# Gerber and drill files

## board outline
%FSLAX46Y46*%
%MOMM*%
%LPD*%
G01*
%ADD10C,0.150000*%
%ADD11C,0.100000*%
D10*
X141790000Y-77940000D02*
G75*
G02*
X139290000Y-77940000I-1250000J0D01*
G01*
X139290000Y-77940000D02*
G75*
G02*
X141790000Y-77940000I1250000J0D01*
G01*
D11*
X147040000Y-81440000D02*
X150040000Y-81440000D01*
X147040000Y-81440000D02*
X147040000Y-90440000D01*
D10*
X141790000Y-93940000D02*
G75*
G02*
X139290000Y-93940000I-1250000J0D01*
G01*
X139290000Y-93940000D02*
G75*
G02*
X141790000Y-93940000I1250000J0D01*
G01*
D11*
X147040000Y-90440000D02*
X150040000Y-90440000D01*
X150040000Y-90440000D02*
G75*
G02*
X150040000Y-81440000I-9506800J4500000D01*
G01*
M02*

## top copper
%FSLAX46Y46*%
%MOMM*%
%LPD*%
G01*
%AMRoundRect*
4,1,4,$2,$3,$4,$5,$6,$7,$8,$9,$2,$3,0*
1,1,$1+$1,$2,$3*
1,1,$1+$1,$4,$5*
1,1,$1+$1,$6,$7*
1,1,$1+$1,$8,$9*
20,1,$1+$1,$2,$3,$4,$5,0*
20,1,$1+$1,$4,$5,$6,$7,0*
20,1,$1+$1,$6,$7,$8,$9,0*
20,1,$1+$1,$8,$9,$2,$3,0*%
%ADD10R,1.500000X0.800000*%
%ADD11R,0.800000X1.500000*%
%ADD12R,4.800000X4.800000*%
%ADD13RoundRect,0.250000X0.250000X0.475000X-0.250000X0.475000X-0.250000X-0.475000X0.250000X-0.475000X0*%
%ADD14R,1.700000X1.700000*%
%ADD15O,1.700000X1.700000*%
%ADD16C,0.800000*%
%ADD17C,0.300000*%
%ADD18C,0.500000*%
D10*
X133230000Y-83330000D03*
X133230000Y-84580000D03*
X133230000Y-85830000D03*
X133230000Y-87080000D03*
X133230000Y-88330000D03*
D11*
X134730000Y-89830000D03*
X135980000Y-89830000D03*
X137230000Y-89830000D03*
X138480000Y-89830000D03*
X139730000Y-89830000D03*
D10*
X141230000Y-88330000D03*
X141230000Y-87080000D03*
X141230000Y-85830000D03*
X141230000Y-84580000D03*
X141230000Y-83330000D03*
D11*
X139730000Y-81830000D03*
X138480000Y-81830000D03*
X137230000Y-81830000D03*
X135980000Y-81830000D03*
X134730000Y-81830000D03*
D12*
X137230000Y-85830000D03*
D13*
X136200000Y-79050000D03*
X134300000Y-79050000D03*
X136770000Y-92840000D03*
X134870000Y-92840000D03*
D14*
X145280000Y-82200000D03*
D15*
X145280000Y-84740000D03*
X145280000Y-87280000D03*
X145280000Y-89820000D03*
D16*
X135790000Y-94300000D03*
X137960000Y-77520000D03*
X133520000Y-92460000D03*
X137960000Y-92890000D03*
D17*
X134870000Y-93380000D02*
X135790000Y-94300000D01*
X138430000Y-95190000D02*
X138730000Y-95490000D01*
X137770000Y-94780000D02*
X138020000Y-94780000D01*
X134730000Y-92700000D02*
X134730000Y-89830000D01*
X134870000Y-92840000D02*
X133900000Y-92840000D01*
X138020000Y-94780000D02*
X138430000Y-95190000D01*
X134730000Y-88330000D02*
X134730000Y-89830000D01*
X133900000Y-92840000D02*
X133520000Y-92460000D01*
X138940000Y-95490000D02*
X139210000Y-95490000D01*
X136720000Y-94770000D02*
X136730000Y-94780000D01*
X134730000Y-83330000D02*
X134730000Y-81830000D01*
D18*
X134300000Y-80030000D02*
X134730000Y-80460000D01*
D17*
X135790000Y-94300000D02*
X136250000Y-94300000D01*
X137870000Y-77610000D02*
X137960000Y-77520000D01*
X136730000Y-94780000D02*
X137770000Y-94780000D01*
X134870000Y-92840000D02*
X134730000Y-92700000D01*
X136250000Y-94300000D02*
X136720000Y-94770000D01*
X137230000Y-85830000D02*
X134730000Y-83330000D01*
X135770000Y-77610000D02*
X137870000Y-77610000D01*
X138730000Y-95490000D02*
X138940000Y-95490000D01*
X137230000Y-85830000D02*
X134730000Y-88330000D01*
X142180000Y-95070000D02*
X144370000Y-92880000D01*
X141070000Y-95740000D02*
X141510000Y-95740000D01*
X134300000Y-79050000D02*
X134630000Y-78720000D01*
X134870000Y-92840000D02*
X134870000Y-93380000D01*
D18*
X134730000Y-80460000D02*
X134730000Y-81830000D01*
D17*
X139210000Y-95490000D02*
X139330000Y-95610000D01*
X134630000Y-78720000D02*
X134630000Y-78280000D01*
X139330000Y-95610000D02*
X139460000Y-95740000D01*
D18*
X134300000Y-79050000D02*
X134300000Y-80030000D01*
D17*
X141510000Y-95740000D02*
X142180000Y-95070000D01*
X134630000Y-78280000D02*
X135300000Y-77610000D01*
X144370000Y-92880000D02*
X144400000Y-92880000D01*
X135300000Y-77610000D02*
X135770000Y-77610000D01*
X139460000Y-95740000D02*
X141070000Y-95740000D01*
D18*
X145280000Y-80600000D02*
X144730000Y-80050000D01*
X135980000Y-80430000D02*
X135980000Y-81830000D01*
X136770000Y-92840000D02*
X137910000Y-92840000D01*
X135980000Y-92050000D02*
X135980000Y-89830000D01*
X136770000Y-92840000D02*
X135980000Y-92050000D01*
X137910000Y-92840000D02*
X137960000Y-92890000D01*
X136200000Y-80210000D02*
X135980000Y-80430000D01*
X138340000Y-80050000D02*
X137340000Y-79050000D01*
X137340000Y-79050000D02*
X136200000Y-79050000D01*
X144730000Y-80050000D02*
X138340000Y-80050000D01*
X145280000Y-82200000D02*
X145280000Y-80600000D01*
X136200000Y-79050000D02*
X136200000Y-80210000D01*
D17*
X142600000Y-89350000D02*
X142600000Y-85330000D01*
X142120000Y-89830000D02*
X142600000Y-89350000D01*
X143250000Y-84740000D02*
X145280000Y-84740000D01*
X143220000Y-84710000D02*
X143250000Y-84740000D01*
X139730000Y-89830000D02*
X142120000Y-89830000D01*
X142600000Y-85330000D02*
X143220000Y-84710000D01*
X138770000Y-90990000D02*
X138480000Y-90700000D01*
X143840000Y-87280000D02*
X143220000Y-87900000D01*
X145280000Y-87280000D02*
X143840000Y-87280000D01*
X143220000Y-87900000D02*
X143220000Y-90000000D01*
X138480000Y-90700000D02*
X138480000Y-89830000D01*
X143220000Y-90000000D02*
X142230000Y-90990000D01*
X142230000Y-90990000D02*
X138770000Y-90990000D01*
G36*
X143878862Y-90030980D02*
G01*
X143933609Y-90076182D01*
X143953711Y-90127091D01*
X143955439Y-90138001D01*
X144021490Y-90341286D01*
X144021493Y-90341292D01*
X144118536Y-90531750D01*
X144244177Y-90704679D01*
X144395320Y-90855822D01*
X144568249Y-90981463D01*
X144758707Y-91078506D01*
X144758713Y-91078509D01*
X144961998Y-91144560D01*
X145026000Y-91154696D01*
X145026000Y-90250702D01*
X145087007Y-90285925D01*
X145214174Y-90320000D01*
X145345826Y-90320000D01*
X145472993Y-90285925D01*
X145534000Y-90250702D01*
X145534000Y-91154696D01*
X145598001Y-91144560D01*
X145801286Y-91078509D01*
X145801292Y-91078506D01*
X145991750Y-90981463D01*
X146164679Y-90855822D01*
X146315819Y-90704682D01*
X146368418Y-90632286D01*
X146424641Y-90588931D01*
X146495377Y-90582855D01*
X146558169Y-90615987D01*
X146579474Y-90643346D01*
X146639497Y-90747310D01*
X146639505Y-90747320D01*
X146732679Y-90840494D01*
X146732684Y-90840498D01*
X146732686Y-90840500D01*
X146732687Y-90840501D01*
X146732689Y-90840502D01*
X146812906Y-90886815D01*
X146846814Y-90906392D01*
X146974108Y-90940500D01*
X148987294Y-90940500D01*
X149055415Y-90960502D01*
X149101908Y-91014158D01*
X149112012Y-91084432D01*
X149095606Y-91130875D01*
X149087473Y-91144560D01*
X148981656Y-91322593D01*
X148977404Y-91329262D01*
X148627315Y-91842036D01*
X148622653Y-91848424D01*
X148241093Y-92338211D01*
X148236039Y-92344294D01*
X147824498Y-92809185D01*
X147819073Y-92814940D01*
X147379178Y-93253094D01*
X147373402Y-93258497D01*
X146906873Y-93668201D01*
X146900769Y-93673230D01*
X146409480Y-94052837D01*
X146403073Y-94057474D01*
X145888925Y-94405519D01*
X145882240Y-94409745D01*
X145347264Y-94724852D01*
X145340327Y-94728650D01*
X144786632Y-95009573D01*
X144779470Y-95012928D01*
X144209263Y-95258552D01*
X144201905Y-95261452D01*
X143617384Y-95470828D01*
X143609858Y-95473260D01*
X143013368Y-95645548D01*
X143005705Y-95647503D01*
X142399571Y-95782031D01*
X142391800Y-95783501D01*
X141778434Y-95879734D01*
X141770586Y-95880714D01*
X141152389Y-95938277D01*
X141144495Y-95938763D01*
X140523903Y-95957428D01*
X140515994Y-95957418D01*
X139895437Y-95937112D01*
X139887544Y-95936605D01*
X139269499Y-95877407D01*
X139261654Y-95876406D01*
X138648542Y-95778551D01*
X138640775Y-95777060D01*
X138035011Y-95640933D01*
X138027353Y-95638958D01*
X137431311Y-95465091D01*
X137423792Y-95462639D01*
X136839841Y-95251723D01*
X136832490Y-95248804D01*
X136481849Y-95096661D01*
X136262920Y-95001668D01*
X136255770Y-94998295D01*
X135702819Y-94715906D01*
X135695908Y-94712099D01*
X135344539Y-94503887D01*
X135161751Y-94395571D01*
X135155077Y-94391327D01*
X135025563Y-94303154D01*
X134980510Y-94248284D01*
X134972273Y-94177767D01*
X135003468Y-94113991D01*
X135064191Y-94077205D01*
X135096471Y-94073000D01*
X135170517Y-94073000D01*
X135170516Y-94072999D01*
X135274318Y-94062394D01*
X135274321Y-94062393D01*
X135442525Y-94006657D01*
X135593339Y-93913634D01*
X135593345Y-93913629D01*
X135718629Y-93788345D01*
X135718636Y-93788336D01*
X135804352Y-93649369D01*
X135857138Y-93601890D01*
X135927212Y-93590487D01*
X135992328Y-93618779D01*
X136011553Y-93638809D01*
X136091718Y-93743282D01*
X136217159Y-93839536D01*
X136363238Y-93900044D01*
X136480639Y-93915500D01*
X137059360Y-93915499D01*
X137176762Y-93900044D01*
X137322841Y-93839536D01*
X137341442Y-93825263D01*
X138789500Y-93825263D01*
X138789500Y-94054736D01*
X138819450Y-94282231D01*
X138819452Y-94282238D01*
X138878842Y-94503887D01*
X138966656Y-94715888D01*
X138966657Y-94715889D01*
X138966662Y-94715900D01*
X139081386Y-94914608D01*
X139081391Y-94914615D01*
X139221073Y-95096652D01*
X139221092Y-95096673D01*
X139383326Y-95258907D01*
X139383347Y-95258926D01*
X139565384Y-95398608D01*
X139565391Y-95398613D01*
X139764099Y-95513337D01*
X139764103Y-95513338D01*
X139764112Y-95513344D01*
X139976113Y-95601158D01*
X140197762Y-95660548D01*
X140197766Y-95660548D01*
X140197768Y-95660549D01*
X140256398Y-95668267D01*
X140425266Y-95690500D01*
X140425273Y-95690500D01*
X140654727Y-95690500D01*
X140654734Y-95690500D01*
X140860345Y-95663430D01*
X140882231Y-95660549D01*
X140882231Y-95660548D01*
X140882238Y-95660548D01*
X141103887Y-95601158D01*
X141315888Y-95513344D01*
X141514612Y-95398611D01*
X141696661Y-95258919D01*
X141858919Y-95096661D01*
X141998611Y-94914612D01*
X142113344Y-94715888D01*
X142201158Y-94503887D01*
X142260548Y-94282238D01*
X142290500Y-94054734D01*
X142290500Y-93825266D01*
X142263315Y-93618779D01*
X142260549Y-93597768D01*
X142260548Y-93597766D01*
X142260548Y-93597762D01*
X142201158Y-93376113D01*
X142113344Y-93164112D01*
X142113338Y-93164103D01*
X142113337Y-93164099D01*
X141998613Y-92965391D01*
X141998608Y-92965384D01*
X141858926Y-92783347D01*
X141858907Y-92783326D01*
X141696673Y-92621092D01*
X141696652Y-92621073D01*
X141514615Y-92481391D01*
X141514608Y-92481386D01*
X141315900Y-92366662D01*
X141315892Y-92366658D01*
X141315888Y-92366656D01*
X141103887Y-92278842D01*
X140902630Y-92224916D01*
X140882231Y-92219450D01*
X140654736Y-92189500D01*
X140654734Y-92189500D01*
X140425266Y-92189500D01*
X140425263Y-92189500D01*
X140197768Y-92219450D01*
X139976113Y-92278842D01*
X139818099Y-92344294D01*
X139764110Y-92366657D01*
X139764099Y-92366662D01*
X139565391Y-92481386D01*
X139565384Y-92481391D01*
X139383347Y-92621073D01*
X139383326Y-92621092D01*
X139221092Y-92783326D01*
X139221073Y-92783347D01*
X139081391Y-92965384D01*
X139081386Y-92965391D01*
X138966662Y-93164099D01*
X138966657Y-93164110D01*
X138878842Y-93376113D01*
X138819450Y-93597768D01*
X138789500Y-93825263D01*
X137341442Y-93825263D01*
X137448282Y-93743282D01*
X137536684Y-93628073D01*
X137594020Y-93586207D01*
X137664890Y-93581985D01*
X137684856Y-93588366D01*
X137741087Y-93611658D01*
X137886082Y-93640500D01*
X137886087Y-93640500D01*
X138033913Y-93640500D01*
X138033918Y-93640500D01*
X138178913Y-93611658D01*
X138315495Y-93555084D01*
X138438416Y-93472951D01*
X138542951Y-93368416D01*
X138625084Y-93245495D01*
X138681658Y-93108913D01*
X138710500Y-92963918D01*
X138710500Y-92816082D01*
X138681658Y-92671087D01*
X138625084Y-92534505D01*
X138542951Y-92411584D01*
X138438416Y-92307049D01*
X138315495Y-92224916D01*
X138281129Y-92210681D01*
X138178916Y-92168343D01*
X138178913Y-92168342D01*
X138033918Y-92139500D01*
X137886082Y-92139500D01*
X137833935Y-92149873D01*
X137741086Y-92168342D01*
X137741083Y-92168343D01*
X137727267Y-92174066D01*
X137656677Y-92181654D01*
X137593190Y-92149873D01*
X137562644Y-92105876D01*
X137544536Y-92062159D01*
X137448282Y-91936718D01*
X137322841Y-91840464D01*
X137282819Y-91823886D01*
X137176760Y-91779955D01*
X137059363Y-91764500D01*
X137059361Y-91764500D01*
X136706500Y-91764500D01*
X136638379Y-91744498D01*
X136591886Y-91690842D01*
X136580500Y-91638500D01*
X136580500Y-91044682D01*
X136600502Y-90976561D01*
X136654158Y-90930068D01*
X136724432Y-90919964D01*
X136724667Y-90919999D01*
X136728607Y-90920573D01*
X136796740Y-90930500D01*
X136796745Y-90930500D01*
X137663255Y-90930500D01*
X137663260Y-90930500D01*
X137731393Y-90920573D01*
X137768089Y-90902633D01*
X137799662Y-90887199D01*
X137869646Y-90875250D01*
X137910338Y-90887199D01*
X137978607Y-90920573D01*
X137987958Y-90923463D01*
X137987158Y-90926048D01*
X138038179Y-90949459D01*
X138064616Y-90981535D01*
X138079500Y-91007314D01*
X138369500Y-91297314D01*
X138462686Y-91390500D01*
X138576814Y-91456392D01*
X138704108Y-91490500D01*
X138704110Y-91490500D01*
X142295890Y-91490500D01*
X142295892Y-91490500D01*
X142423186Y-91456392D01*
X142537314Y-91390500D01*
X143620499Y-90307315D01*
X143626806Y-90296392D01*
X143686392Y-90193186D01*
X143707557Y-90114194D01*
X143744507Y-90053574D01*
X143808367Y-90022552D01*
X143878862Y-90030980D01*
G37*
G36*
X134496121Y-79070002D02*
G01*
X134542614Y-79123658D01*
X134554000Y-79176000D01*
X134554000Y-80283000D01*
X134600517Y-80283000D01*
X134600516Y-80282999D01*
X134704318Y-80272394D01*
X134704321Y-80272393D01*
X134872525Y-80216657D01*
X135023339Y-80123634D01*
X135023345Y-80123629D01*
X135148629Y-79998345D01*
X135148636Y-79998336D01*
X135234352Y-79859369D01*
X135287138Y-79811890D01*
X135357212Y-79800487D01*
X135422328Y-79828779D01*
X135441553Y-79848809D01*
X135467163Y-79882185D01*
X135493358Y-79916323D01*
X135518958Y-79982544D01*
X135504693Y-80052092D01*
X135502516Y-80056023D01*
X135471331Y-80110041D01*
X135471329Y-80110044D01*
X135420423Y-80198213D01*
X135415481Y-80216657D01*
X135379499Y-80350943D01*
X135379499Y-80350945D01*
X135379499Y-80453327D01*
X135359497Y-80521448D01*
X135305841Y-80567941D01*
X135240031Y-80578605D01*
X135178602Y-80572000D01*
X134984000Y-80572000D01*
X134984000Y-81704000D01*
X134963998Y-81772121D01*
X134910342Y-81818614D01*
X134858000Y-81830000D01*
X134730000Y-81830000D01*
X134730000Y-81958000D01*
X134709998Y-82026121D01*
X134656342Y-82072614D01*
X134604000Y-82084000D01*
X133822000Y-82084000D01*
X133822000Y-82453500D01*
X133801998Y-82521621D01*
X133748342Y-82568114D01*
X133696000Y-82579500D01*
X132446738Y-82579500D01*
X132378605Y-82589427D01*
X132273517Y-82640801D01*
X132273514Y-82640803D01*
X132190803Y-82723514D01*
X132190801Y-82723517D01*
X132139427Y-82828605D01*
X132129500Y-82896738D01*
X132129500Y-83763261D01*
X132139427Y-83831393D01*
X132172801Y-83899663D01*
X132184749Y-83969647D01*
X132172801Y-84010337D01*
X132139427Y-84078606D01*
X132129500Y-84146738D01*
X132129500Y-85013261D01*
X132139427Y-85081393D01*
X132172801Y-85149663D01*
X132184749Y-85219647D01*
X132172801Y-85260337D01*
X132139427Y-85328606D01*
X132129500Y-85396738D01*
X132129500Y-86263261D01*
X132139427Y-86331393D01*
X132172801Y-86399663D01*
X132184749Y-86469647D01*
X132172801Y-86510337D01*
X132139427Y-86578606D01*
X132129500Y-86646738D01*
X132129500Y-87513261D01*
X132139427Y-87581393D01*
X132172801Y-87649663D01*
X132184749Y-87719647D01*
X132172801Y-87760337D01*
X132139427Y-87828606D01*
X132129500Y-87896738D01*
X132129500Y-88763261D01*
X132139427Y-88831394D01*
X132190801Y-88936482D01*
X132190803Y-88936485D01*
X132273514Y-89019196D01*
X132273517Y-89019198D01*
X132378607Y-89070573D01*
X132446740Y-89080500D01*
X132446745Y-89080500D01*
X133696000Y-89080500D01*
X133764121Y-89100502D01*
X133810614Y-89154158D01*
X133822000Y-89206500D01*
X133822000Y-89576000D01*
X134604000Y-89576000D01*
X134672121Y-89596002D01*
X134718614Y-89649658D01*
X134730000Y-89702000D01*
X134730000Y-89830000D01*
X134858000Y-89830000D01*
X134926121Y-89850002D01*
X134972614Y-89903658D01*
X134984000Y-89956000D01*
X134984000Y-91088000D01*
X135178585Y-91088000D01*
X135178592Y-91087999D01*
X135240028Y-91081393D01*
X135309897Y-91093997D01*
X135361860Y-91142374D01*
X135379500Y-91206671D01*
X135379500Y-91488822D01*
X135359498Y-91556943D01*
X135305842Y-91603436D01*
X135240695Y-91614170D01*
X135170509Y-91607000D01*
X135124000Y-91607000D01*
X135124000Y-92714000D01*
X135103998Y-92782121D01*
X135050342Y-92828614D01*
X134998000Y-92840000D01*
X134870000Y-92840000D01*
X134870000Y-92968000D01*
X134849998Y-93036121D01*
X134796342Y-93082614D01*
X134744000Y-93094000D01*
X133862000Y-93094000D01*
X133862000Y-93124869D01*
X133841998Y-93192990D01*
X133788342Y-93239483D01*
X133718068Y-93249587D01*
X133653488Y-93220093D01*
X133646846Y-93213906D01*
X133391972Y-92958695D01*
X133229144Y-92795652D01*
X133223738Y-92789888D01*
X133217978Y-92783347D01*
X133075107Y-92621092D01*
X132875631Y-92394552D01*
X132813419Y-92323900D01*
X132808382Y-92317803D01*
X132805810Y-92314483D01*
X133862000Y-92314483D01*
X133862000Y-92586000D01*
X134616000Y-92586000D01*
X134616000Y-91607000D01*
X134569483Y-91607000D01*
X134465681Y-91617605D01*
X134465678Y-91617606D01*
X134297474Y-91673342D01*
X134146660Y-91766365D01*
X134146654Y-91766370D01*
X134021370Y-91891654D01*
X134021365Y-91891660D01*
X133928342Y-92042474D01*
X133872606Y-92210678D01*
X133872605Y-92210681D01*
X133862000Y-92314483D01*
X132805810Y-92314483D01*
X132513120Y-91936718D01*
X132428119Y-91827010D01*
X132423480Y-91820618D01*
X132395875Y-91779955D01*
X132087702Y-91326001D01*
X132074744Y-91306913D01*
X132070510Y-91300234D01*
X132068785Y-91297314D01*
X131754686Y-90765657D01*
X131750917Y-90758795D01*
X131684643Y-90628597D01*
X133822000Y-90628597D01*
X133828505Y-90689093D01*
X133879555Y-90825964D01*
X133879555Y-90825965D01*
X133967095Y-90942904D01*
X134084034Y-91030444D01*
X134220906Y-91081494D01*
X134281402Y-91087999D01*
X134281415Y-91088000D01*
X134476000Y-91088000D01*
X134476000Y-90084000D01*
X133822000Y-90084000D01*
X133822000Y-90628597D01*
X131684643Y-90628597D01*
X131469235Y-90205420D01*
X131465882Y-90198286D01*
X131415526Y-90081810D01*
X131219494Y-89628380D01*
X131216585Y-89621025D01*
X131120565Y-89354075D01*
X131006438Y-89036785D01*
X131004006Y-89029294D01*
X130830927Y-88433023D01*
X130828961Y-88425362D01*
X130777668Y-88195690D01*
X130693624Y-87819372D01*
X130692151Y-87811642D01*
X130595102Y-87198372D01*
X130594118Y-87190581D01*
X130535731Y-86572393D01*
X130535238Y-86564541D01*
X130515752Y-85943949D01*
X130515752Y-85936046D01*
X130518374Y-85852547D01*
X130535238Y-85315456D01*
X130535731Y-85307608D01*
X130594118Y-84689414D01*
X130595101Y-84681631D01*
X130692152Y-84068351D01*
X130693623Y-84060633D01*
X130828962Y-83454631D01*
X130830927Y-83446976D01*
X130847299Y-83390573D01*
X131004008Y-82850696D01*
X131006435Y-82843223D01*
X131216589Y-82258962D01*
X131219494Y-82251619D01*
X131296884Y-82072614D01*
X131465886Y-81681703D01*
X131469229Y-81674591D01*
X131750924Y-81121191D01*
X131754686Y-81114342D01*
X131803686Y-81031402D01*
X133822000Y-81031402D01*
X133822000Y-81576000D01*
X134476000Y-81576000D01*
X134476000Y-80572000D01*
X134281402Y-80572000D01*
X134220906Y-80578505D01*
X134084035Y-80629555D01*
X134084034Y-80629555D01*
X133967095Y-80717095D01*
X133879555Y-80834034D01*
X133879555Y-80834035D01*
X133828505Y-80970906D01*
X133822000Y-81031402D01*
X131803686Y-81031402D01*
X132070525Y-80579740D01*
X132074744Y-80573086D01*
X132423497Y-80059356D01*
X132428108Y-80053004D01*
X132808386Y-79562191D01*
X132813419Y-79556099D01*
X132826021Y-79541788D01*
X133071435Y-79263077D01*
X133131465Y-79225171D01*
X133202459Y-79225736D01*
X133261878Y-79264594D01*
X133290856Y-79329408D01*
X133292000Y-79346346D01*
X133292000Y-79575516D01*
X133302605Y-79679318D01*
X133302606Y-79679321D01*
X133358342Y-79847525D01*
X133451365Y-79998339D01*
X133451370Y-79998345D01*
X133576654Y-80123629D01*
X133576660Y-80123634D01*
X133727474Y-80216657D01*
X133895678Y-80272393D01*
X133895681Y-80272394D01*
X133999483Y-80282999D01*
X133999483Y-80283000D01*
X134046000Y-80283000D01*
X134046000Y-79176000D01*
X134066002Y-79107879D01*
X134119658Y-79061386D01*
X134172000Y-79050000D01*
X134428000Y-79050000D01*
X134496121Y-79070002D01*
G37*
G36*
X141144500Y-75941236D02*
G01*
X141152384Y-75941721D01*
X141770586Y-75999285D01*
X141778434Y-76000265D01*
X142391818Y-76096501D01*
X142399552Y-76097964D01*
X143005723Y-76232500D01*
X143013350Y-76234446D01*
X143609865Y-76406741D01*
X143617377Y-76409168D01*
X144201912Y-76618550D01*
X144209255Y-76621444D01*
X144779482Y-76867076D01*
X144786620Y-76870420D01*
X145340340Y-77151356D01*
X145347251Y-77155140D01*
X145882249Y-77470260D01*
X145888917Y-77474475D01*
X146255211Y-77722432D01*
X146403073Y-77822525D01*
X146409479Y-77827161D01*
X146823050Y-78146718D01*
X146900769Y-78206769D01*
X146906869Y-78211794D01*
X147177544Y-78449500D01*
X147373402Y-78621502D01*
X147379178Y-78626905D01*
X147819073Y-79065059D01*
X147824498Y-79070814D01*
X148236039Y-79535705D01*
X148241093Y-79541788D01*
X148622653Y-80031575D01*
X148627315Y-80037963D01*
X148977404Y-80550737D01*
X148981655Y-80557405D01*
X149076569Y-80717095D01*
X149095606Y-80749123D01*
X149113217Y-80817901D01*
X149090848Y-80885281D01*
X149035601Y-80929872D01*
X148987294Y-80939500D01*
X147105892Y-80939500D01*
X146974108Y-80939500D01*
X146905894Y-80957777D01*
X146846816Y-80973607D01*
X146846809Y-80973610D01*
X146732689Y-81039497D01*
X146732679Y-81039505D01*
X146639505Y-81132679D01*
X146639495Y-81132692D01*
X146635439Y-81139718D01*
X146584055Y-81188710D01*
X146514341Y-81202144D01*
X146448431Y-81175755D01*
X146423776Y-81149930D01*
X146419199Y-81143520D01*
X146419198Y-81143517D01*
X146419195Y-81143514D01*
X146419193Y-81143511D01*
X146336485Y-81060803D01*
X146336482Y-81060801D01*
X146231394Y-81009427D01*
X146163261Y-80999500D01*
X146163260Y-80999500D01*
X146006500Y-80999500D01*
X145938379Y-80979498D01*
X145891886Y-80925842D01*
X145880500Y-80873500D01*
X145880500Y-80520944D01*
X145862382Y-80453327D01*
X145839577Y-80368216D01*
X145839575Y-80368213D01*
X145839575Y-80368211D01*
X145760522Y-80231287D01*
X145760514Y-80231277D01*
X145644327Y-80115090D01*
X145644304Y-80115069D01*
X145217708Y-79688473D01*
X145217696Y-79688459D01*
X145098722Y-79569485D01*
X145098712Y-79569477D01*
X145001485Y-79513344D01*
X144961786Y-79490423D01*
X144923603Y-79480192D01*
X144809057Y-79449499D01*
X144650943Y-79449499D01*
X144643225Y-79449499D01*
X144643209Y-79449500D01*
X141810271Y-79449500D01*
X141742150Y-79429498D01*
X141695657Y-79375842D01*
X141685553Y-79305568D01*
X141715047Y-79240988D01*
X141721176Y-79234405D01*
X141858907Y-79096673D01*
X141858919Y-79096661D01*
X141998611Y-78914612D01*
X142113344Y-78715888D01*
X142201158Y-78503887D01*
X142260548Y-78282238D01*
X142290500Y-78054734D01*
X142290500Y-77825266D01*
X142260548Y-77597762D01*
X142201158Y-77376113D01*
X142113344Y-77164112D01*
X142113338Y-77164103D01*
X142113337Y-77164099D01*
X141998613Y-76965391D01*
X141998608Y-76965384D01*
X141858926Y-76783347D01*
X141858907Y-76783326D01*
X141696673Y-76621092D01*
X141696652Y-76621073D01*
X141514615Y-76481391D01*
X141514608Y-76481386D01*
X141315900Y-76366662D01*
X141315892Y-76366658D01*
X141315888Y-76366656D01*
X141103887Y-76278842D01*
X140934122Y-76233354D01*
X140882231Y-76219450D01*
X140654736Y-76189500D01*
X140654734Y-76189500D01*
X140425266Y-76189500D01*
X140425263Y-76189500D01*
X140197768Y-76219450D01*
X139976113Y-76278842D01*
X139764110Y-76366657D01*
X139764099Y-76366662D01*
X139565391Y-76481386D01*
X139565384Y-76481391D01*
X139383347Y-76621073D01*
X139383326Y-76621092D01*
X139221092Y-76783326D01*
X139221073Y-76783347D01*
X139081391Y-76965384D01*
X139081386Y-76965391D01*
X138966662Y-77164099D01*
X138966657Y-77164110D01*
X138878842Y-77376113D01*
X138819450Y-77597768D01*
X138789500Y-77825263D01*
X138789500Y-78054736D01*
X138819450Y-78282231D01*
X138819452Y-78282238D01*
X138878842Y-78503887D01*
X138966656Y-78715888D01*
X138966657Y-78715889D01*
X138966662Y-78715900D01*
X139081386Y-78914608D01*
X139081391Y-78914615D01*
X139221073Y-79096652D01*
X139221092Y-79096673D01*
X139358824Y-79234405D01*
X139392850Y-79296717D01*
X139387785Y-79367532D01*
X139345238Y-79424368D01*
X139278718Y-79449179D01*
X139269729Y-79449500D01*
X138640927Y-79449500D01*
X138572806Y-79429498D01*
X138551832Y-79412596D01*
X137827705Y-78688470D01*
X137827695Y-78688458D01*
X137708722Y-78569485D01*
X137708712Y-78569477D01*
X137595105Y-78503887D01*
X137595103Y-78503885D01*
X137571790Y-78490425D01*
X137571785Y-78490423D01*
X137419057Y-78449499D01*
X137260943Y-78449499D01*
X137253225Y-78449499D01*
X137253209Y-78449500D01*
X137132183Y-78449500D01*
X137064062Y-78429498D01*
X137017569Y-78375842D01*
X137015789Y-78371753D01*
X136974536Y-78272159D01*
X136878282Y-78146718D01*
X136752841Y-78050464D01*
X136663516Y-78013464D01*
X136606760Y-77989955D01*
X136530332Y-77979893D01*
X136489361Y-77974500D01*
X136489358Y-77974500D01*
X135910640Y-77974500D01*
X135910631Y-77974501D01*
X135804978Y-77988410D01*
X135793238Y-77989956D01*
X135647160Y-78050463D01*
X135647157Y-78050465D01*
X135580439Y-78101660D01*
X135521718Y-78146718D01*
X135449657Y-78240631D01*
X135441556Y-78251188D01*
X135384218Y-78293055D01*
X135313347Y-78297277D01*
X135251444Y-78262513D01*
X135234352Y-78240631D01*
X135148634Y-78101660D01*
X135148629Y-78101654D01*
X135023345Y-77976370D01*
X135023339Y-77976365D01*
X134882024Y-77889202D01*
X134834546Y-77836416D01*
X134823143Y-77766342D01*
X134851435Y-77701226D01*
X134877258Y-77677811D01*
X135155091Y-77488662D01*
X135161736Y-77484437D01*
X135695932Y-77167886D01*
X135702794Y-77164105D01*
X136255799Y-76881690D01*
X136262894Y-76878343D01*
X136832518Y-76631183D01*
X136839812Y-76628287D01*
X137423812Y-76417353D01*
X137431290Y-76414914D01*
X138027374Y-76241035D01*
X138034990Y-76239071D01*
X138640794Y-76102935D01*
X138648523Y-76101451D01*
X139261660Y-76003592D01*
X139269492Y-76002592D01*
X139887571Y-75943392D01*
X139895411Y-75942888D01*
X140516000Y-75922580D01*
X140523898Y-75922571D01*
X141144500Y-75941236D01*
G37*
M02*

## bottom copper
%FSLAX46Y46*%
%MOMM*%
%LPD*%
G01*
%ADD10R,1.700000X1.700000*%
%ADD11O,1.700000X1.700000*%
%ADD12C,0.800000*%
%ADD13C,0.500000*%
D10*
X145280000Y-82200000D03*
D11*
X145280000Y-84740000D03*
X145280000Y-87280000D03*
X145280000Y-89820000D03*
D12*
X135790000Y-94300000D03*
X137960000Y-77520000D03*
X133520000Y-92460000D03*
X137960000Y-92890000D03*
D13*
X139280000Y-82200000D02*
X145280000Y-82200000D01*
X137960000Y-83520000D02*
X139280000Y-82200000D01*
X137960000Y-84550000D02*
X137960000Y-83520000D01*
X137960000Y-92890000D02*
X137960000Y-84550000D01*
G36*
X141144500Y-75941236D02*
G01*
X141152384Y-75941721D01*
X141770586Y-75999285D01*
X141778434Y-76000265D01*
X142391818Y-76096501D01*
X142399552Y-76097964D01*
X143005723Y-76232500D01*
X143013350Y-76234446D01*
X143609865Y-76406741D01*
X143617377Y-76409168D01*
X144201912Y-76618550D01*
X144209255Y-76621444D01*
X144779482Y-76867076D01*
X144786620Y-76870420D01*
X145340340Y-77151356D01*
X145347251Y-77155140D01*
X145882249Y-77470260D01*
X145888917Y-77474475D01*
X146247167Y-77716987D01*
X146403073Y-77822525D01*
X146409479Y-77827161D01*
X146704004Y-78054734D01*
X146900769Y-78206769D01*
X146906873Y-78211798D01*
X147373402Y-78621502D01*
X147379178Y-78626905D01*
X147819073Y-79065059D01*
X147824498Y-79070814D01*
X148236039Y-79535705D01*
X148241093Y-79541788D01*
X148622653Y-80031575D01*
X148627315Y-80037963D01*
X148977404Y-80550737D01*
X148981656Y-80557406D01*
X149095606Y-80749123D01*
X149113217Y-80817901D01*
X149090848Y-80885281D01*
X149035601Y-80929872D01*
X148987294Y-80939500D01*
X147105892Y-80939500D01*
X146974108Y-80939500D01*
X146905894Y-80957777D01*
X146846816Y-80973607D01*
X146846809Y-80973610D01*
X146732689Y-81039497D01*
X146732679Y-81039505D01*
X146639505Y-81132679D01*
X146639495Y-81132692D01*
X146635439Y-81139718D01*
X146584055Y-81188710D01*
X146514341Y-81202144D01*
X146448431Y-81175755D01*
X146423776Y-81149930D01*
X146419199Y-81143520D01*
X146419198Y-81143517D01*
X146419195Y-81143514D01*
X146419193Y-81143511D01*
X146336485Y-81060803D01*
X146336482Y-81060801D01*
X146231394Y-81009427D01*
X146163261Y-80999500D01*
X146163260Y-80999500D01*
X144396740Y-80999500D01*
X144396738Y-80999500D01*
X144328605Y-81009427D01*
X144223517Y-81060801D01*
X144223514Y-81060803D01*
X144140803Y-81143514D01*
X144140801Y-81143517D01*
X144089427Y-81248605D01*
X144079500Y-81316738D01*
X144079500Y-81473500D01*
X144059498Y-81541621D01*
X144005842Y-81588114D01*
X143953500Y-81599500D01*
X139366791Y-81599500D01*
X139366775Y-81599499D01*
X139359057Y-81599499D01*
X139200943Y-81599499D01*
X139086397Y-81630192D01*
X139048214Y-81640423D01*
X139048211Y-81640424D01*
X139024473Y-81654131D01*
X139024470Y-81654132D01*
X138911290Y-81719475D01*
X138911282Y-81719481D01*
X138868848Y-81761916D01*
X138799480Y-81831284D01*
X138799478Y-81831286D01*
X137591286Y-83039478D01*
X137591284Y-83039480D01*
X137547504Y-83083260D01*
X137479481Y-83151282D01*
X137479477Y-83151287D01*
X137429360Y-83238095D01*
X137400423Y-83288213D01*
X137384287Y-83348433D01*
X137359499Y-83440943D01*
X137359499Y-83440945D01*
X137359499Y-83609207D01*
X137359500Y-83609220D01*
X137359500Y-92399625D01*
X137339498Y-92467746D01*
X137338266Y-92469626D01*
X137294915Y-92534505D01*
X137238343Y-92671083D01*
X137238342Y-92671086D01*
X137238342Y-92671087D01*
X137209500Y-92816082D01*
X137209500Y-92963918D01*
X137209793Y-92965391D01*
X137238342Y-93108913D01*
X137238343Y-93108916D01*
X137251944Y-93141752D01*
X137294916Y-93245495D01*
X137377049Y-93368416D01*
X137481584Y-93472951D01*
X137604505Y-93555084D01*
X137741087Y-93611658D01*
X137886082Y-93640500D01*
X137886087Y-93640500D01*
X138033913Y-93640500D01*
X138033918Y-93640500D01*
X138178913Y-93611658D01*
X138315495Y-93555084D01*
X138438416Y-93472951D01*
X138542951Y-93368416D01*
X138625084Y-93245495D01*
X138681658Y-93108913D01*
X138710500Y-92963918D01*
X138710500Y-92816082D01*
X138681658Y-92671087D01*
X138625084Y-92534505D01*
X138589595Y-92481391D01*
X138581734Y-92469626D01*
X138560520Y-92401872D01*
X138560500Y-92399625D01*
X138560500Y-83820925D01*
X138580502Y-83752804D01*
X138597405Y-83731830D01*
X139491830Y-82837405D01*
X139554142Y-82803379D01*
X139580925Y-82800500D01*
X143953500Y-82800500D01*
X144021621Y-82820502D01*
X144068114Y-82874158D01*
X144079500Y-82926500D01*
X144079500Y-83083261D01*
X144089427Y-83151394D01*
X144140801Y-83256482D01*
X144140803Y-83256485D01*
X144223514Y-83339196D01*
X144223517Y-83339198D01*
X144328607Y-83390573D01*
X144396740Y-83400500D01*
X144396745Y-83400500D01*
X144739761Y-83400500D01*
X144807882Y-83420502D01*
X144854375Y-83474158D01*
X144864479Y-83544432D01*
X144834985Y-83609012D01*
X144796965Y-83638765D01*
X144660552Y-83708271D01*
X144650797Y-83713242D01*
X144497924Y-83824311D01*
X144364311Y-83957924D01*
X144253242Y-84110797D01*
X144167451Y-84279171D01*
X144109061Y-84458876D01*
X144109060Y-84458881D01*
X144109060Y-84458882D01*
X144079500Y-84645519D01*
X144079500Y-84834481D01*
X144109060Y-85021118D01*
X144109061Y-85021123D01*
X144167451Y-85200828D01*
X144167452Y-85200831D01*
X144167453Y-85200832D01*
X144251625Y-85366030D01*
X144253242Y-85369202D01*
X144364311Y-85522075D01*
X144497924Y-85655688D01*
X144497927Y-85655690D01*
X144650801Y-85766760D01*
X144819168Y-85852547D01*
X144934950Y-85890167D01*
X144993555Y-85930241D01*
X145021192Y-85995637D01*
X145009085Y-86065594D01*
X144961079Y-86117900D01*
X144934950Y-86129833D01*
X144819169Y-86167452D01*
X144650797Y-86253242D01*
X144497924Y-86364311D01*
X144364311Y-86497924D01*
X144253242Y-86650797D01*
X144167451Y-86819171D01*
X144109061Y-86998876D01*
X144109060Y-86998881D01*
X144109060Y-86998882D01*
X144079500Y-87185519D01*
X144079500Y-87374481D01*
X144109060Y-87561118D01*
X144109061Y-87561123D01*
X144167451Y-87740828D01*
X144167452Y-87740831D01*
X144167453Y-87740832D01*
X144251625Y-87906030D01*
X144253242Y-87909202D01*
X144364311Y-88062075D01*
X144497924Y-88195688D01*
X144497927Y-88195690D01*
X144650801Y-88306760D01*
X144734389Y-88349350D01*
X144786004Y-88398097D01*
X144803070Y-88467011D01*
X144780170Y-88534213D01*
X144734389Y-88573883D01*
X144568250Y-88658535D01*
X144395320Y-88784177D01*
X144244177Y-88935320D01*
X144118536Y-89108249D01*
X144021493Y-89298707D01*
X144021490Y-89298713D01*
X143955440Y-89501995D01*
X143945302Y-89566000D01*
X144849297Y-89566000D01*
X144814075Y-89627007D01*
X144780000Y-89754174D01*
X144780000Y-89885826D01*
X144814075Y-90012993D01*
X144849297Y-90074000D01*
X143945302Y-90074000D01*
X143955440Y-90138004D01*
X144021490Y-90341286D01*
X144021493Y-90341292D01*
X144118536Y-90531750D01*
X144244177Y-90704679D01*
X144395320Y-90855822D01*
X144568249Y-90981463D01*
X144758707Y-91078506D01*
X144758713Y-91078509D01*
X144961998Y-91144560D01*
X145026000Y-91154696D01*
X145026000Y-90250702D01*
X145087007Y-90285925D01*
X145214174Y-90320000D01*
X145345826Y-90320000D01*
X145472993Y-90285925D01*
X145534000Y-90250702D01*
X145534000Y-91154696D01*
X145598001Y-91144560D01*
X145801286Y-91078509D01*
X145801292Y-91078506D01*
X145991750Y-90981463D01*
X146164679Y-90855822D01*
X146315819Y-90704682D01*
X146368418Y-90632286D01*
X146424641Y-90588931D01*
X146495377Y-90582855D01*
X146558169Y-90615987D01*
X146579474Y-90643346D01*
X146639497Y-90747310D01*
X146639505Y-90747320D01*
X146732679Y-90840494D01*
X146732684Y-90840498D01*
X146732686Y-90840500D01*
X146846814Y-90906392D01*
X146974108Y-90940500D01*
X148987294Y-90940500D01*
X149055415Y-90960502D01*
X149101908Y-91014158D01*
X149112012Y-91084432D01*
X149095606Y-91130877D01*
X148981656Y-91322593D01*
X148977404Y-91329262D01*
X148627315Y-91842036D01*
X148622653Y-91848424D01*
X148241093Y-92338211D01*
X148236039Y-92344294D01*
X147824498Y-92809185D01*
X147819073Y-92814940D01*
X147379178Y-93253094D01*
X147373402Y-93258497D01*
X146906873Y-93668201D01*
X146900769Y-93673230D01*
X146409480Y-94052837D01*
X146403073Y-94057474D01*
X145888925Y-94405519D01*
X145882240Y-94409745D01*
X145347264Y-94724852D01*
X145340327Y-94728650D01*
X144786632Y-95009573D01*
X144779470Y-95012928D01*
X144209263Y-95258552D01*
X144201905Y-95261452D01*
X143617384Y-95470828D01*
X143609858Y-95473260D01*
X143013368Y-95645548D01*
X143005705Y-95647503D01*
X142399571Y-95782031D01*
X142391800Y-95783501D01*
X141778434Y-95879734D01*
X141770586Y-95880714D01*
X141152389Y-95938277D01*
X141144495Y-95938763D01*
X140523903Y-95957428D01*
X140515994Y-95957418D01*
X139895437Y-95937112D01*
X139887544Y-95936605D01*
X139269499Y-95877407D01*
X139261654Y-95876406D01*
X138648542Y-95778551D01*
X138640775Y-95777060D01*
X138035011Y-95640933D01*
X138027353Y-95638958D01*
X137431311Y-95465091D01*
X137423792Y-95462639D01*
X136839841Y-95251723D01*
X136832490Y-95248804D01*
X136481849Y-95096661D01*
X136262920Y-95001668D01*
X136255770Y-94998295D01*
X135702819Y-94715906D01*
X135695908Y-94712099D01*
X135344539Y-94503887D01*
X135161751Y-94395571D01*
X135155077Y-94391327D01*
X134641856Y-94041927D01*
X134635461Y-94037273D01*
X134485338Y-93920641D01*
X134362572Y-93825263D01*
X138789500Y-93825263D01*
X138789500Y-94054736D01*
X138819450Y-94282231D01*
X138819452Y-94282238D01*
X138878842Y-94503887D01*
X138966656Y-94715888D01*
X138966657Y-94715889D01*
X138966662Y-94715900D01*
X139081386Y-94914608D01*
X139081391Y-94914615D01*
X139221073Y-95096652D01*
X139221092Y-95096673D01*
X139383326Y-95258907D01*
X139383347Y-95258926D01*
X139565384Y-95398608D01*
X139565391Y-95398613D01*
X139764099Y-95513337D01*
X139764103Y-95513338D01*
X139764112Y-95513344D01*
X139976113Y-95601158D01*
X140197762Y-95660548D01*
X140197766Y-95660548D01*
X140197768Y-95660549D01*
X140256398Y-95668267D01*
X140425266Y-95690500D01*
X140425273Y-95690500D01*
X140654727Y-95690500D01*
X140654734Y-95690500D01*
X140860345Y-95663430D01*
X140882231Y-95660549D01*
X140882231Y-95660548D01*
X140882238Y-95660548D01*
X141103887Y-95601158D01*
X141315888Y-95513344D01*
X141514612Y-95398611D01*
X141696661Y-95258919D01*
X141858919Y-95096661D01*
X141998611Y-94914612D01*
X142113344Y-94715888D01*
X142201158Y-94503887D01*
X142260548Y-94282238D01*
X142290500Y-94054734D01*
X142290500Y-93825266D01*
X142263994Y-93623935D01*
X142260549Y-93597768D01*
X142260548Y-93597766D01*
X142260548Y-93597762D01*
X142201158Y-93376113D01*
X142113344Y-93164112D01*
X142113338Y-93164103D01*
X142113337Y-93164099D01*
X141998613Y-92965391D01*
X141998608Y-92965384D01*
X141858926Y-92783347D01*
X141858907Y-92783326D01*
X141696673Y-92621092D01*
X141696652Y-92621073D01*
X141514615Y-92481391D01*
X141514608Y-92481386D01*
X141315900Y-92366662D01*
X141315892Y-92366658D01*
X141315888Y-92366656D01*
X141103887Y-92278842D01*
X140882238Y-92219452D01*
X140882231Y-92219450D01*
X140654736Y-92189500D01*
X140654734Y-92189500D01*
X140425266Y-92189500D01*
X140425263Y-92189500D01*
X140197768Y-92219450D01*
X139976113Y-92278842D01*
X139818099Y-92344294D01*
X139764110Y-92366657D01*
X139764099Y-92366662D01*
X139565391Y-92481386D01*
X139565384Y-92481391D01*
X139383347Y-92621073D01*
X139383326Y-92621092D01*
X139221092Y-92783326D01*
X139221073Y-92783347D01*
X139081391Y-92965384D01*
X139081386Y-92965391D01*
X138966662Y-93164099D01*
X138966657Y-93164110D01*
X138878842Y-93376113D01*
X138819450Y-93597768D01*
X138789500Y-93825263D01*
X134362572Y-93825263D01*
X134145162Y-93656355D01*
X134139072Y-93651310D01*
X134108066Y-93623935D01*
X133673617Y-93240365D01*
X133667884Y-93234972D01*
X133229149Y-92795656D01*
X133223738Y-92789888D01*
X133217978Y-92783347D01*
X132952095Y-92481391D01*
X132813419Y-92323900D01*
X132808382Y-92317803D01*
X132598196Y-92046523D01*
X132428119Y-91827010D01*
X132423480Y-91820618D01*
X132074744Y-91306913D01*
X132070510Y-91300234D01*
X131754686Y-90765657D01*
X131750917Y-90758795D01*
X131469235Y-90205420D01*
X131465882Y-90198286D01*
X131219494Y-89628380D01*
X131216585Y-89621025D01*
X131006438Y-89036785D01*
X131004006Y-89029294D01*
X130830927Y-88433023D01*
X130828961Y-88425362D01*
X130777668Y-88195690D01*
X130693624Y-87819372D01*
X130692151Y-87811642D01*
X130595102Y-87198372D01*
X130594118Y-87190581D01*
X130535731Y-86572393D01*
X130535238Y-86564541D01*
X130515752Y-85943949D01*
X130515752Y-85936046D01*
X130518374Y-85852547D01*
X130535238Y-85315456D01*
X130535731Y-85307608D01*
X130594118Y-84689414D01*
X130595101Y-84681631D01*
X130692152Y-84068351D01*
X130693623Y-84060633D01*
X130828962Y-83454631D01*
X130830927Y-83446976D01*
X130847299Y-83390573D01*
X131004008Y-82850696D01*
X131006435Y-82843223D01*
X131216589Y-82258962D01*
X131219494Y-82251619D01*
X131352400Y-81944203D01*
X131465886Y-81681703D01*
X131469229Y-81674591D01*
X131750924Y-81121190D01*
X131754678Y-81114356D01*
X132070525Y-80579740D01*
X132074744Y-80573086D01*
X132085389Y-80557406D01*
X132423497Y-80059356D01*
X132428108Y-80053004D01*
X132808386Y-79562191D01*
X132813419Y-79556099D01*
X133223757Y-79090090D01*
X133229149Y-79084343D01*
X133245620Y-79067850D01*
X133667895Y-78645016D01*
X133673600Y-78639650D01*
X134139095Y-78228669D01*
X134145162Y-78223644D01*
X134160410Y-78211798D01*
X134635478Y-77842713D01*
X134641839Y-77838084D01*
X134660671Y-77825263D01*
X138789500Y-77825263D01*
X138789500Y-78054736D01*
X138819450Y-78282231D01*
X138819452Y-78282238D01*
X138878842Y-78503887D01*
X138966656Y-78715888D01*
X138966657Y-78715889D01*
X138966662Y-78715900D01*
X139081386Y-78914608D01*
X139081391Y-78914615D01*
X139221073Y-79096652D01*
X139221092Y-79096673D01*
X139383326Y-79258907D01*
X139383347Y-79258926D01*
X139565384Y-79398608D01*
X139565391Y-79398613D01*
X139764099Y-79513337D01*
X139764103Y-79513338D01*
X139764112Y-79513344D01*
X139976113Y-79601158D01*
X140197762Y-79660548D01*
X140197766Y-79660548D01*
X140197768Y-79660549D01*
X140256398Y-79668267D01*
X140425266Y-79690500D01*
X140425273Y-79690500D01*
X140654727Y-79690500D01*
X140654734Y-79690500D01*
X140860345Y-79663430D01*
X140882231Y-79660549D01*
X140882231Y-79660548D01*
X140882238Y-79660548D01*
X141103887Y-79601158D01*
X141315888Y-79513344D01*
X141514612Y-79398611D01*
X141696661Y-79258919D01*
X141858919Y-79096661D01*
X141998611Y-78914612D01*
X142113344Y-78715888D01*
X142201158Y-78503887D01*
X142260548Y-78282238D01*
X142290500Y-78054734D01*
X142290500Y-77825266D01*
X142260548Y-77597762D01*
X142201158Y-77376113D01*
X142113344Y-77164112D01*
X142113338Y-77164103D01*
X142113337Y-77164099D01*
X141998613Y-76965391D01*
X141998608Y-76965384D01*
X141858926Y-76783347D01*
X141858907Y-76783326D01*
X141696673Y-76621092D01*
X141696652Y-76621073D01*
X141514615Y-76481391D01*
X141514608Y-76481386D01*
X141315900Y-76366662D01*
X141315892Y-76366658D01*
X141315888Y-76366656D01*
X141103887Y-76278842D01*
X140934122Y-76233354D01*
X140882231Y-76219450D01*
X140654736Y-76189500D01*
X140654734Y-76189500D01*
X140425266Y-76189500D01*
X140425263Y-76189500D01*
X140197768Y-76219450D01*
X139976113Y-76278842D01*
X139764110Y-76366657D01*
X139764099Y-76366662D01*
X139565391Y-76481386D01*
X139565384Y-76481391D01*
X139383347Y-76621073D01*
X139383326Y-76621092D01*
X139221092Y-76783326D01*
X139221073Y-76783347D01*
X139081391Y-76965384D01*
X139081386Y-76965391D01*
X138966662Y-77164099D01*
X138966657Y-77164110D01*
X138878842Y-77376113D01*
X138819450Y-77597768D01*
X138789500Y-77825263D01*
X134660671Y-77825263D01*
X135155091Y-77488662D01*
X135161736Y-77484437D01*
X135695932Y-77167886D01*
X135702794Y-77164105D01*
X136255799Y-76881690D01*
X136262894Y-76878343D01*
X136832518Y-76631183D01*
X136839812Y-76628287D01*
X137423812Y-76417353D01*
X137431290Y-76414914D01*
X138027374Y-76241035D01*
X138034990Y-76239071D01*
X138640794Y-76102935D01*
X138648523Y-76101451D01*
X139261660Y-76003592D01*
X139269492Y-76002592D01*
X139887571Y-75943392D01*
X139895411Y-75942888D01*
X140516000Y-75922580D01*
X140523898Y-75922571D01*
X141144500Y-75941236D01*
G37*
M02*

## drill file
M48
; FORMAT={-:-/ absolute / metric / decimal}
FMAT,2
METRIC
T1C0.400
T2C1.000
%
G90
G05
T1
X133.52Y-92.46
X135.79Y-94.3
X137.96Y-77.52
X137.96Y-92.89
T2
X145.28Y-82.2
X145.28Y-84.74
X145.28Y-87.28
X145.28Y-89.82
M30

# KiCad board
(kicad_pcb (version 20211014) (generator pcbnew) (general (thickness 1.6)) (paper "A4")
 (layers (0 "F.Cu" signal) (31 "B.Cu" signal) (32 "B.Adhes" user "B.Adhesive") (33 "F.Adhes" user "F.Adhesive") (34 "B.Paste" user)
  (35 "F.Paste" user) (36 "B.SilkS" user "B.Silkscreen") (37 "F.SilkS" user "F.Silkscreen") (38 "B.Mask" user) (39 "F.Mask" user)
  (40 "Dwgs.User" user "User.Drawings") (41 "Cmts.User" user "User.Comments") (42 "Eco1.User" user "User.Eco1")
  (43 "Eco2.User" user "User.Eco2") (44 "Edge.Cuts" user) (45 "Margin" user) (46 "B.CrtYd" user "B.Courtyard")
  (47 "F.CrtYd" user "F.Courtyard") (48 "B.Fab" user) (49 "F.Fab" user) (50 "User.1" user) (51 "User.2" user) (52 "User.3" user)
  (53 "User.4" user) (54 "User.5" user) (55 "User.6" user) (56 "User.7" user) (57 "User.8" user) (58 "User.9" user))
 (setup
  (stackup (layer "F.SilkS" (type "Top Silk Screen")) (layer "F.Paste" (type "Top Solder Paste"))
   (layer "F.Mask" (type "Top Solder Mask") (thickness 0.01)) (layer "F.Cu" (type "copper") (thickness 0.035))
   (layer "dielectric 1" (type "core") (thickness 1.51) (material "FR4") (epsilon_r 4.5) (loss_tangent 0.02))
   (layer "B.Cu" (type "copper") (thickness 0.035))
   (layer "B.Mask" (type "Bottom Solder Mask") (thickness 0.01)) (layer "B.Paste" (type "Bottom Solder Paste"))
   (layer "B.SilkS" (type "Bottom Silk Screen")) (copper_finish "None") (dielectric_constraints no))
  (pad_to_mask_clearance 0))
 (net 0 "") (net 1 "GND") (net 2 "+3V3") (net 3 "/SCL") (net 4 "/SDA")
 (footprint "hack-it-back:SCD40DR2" (layer "F.Cu") (at 137.23 85.83)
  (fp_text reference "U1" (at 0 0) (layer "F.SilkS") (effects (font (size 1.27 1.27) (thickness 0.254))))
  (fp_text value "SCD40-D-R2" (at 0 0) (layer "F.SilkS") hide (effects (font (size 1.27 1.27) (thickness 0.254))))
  (pad "1" smd rect (at -4 -2.5 90) (size 0.8 1.5) (layers "F.Cu" "F.Paste" "F.Mask"))
  (pad "2" smd rect (at -4 -1.25 90) (size 0.8 1.5) (layers "F.Cu" "F.Paste" "F.Mask"))
  (pad "3" smd rect (at -4 0 90) (size 0.8 1.5) (layers "F.Cu" "F.Paste" "F.Mask"))
  (pad "4" smd rect (at -4 1.25 90) (size 0.8 1.5) (layers "F.Cu" "F.Paste" "F.Mask"))
  (pad "5" smd rect (at -4 2.5 90) (size 0.8 1.5) (layers "F.Cu" "F.Paste" "F.Mask"))
  (pad "6" smd rect (at -2.5 4) (size 0.8 1.5) (layers "F.Cu" "F.Paste" "F.Mask") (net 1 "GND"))
  (pad "7" smd rect (at -1.25 4) (size 0.8 1.5) (layers "F.Cu" "F.Paste" "F.Mask") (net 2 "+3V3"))
  (pad "8" smd rect (at 0 4) (size 0.8 1.5) (layers "F.Cu" "F.Paste" "F.Mask"))
  (pad "9" smd rect (at 1.25 4) (size 0.8 1.5) (layers "F.Cu" "F.Paste" "F.Mask") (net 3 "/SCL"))
  (pad "10" smd rect (at 2.5 4) (size 0.8 1.5) (layers "F.Cu" "F.Paste" "F.Mask") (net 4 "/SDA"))
  (pad "11" smd rect (at 4 2.5 90) (size 0.8 1.5) (layers "F.Cu" "F.Paste" "F.Mask"))
  (pad "12" smd rect (at 4 1.25 90) (size 0.8 1.5) (layers "F.Cu" "F.Paste" "F.Mask"))
  (pad "13" smd rect (at 4 0 90) (size 0.8 1.5) (layers "F.Cu" "F.Paste" "F.Mask"))
  (pad "14" smd rect (at 4 -1.25 90) (size 0.8 1.5) (layers "F.Cu" "F.Paste" "F.Mask"))
  (pad "15" smd rect (at 4 -2.5 90) (size 0.8 1.5) (layers "F.Cu" "F.Paste" "F.Mask"))
  (pad "16" smd rect (at 2.5 -4) (size 0.8 1.5) (layers "F.Cu" "F.Paste" "F.Mask"))
  (pad "17" smd rect (at 1.25 -4) (size 0.8 1.5) (layers "F.Cu" "F.Paste" "F.Mask"))
  (pad "18" smd rect (at 0 -4) (size 0.8 1.5) (layers "F.Cu" "F.Paste" "F.Mask"))
  (pad "19" smd rect (at -1.25 -4) (size 0.8 1.5) (layers "F.Cu" "F.Paste" "F.Mask") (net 2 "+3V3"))
  (pad "20" smd rect (at -2.5 -4) (size 0.8 1.5) (layers "F.Cu" "F.Paste" "F.Mask") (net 1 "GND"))
  (pad "21" smd rect (at 0 0) (size 4.8 4.8) (layers "F.Cu" "F.Paste" "F.Mask") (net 1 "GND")))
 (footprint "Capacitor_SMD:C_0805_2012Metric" (layer "F.Cu") (at 135.25 79.05 180)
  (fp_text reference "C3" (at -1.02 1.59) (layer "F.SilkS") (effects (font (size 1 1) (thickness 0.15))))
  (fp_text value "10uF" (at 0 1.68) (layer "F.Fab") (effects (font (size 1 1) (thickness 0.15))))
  (pad "1" smd roundrect locked (at -0.95 0 180) (size 1 1.45) (layers "F.Cu" "F.Paste" "F.Mask") (roundrect_rratio 0.25) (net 2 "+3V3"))
  (pad "2" smd roundrect locked (at 0.95 0 180) (size 1 1.45) (layers "F.Cu" "F.Paste" "F.Mask") (roundrect_rratio 0.25) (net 1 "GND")))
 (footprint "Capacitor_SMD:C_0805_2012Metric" (layer "F.Cu") (at 135.82 92.84 180)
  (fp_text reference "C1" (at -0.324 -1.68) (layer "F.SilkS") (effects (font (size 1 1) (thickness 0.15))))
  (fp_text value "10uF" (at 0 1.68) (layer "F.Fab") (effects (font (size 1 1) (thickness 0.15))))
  (pad "1" smd roundrect locked (at -0.95 0 180) (size 1 1.45) (layers "F.Cu" "F.Paste" "F.Mask") (roundrect_rratio 0.25) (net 2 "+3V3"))
  (pad "2" smd roundrect locked (at 0.95 0 180) (size 1 1.45) (layers "F.Cu" "F.Paste" "F.Mask") (roundrect_rratio 0.25) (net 1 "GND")))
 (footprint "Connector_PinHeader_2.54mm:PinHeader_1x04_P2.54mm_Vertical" (layer "B.Cu") (at 145.28 82.2 180)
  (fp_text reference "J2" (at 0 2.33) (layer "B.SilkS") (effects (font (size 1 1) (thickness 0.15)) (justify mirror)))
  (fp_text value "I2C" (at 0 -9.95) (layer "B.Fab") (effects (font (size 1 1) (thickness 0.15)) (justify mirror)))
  (pad "1" thru_hole rect locked (at 0 0 180) (size 1.7 1.7) (drill 1) (layers *.Cu *.Mask) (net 2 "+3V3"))
  (pad "2" thru_hole oval locked (at 0 -2.54 180) (size 1.7 1.7) (drill 1) (layers *.Cu *.Mask) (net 4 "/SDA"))
  (pad "3" thru_hole oval locked (at 0 -5.08 180) (size 1.7 1.7) (drill 1) (layers *.Cu *.Mask) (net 3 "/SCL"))
  (pad "4" thru_hole oval locked (at 0 -7.62 180) (size 1.7 1.7) (drill 1) (layers *.Cu *.Mask) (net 1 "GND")))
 (gr_circle (center 140.54 77.94) (end 141.79 77.94) (layer "Edge.Cuts") (width 0.15) (fill none))
 (gr_line (start 147.04 81.44) (end 150.04 81.44) (layer "Edge.Cuts") (width 0.1))
 (gr_line (start 147.04 81.44) (end 147.04 90.44) (layer "Edge.Cuts") (width 0.1))
 (gr_circle (center 140.54 93.94) (end 141.79 93.94) (layer "Edge.Cuts") (width 0.15) (fill none))
 (gr_line (start 147.04 90.44) (end 150.04 90.44) (layer "Edge.Cuts") (width 0.1))
 (gr_arc (start 150.04 90.44) (mid 130.015128 85.94) (end 150.04 81.44) (layer "Edge.Cuts") (width 0.1))
 (segment (start 134.87 93.38) (end 135.79 94.3) (width 0.3) (layer "F.Cu") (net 1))
 (segment (start 138.43 95.19) (end 138.73 95.49) (width 0.3) (layer "F.Cu") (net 1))
 (segment (start 137.77 94.78) (end 138.02 94.78) (width 0.3) (layer "F.Cu") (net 1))
 (segment (start 134.73 92.7) (end 134.73 89.83) (width 0.3) (layer "F.Cu") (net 1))
 (segment (start 134.87 92.84) (end 133.9 92.84) (width 0.3) (layer "F.Cu") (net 1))
 (segment (start 138.02 94.78) (end 138.43 95.19) (width 0.3) (layer "F.Cu") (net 1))
 (segment (start 134.73 88.33) (end 134.73 89.83) (width 0.3) (layer "F.Cu") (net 1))
 (segment (start 133.9 92.84) (end 133.52 92.46) (width 0.3) (layer "F.Cu") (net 1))
 (segment (start 138.94 95.49) (end 139.21 95.49) (width 0.3) (layer "F.Cu") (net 1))
 (segment (start 136.72 94.77) (end 136.73 94.78) (width 0.3) (layer "F.Cu") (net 1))
 (segment (start 134.73 83.33) (end 134.73 81.83) (width 0.3) (layer "F.Cu") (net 1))
 (segment (start 134.3 80.03) (end 134.73 80.46) (width 0.5) (layer "F.Cu") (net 1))
 (segment (start 135.79 94.3) (end 136.25 94.3) (width 0.3) (layer "F.Cu") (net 1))
 (segment (start 137.87 77.61) (end 137.96 77.52) (width 0.3) (layer "F.Cu") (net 1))
 (segment (start 136.73 94.78) (end 137.77 94.78) (width 0.3) (layer "F.Cu") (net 1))
 (segment (start 134.87 92.84) (end 134.73 92.7) (width 0.3) (layer "F.Cu") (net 1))
 (segment (start 136.25 94.3) (end 136.72 94.77) (width 0.3) (layer "F.Cu") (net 1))
 (segment (start 137.23 85.83) (end 134.73 83.33) (width 0.3) (layer "F.Cu") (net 1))
 (segment (start 135.77 77.61) (end 137.87 77.61) (width 0.3) (layer "F.Cu") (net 1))
 (segment (start 138.73 95.49) (end 138.94 95.49) (width 0.3) (layer "F.Cu") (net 1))
 (segment (start 137.23 85.83) (end 134.73 88.33) (width 0.3) (layer "F.Cu") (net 1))
 (segment (start 142.18 95.07) (end 144.37 92.88) (width 0.3) (layer "F.Cu") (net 1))
 (segment (start 141.07 95.74) (end 141.51 95.74) (width 0.3) (layer "F.Cu") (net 1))
 (segment (start 134.3 79.05) (end 134.63 78.72) (width 0.3) (layer "F.Cu") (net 1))
 (segment (start 134.87 92.84) (end 134.87 93.38) (width 0.3) (layer "F.Cu") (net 1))
 (segment (start 134.73 80.46) (end 134.73 81.83) (width 0.5) (layer "F.Cu") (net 1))
 (segment (start 139.21 95.49) (end 139.33 95.61) (width 0.3) (layer "F.Cu") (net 1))
 (segment (start 134.63 78.72) (end 134.63 78.28) (width 0.3) (layer "F.Cu") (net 1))
 (segment (start 139.33 95.61) (end 139.46 95.74) (width 0.3) (layer "F.Cu") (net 1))
 (segment (start 134.3 79.05) (end 134.3 80.03) (width 0.5) (layer "F.Cu") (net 1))
 (segment (start 141.51 95.74) (end 142.18 95.07) (width 0.3) (layer "F.Cu") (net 1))
 (segment (start 134.63 78.28) (end 135.3 77.61) (width 0.3) (layer "F.Cu") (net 1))
 (segment (start 144.37 92.88) (end 144.4 92.88) (width 0.3) (layer "F.Cu") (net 1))
 (segment (start 135.3 77.61) (end 135.77 77.61) (width 0.3) (layer "F.Cu") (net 1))
 (segment (start 139.46 95.74) (end 141.07 95.74) (width 0.3) (layer "F.Cu") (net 1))
 (via (at 135.79 94.3) (size 0.8) (drill 0.4) (layers "F.Cu" "B.Cu") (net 1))
 (via (at 137.96 77.52) (size 0.8) (drill 0.4) (layers "F.Cu" "B.Cu") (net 1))
 (via (at 133.52 92.46) (size 0.8) (drill 0.4) (layers "F.Cu" "B.Cu") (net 1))
 (segment (start 145.28 80.6) (end 144.73 80.05) (width 0.5) (layer "F.Cu") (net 2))
 (segment (start 135.98 80.43) (end 135.98 81.83) (width 0.5) (layer "F.Cu") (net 2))
 (segment (start 136.77 92.84) (end 137.91 92.84) (width 0.5) (layer "F.Cu") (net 2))
 (segment (start 135.98 92.05) (end 135.98 89.83) (width 0.5) (layer "F.Cu") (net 2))
 (segment (start 136.77 92.84) (end 135.98 92.05) (width 0.5) (layer "F.Cu") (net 2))
 (segment (start 137.91 92.84) (end 137.96 92.89) (width 0.5) (layer "F.Cu") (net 2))
 (segment (start 136.2 80.21) (end 135.98 80.43) (width 0.5) (layer "F.Cu") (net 2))
 (segment (start 138.34 80.05) (end 137.34 79.05) (width 0.5) (layer "F.Cu") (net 2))
 (segment (start 137.34 79.05) (end 136.2 79.05) (width 0.5) (layer "F.Cu") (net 2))
 (segment (start 144.73 80.05) (end 138.34 80.05) (width 0.5) (layer "F.Cu") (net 2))
 (segment (start 145.28 82.2) (end 145.28 80.6) (width 0.5) (layer "F.Cu") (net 2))
 (segment (start 136.2 79.05) (end 136.2 80.21) (width 0.5) (layer "F.Cu") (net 2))
 (via (at 137.96 92.89) (size 0.8) (drill 0.4) (layers "F.Cu" "B.Cu") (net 2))
 (segment (start 139.28 82.2) (end 145.28 82.2) (width 0.5) (layer "B.Cu") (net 2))
 (segment (start 137.96 83.52) (end 139.28 82.2) (width 0.5) (layer "B.Cu") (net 2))
 (segment (start 137.96 84.55) (end 137.96 83.52) (width 0.5) (layer "B.Cu") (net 2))
 (segment (start 137.96 92.89) (end 137.96 84.55) (width 0.5) (layer "B.Cu") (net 2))
 (segment (start 142.6 89.35) (end 142.6 85.33) (width 0.3) (layer "F.Cu") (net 4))
 (segment (start 142.12 89.83) (end 142.6 89.35) (width 0.3) (layer "F.Cu") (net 4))
 (segment (start 143.25 84.74) (end 145.28 84.74) (width 0.3) (layer "F.Cu") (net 4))
 (segment (start 143.22 84.71) (end 143.25 84.74) (width 0.3) (layer "F.Cu") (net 4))
 (segment (start 139.73 89.83) (end 142.12 89.83) (width 0.3) (layer "F.Cu") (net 4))
 (segment (start 142.6 85.33) (end 143.22 84.71) (width 0.3) (layer "F.Cu") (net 4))
 (segment (start 138.77 90.99) (end 138.48 90.7) (width 0.3) (layer "F.Cu") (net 3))
 (segment (start 143.84 87.28) (end 143.22 87.9) (width 0.3) (layer "F.Cu") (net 3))
 (segment (start 145.28 87.28) (end 143.84 87.28) (width 0.3) (layer "F.Cu") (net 3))
 (segment (start 143.22 87.9) (end 143.22 90) (width 0.3) (layer "F.Cu") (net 3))
 (segment (start 138.48 90.7) (end 138.48 89.83) (width 0.3) (layer "F.Cu") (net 3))
 (segment (start 143.22 90) (end 142.23 90.99) (width 0.3) (layer "F.Cu") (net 3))
 (segment (start 142.23 90.99) (end 138.77 90.99) (width 0.3) (layer "F.Cu") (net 3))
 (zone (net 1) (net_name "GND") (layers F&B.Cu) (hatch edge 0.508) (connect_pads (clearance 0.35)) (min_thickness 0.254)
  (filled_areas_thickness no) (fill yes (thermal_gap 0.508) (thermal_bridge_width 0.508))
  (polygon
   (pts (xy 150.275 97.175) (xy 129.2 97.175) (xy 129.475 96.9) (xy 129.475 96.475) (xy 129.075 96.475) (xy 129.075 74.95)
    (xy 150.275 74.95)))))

